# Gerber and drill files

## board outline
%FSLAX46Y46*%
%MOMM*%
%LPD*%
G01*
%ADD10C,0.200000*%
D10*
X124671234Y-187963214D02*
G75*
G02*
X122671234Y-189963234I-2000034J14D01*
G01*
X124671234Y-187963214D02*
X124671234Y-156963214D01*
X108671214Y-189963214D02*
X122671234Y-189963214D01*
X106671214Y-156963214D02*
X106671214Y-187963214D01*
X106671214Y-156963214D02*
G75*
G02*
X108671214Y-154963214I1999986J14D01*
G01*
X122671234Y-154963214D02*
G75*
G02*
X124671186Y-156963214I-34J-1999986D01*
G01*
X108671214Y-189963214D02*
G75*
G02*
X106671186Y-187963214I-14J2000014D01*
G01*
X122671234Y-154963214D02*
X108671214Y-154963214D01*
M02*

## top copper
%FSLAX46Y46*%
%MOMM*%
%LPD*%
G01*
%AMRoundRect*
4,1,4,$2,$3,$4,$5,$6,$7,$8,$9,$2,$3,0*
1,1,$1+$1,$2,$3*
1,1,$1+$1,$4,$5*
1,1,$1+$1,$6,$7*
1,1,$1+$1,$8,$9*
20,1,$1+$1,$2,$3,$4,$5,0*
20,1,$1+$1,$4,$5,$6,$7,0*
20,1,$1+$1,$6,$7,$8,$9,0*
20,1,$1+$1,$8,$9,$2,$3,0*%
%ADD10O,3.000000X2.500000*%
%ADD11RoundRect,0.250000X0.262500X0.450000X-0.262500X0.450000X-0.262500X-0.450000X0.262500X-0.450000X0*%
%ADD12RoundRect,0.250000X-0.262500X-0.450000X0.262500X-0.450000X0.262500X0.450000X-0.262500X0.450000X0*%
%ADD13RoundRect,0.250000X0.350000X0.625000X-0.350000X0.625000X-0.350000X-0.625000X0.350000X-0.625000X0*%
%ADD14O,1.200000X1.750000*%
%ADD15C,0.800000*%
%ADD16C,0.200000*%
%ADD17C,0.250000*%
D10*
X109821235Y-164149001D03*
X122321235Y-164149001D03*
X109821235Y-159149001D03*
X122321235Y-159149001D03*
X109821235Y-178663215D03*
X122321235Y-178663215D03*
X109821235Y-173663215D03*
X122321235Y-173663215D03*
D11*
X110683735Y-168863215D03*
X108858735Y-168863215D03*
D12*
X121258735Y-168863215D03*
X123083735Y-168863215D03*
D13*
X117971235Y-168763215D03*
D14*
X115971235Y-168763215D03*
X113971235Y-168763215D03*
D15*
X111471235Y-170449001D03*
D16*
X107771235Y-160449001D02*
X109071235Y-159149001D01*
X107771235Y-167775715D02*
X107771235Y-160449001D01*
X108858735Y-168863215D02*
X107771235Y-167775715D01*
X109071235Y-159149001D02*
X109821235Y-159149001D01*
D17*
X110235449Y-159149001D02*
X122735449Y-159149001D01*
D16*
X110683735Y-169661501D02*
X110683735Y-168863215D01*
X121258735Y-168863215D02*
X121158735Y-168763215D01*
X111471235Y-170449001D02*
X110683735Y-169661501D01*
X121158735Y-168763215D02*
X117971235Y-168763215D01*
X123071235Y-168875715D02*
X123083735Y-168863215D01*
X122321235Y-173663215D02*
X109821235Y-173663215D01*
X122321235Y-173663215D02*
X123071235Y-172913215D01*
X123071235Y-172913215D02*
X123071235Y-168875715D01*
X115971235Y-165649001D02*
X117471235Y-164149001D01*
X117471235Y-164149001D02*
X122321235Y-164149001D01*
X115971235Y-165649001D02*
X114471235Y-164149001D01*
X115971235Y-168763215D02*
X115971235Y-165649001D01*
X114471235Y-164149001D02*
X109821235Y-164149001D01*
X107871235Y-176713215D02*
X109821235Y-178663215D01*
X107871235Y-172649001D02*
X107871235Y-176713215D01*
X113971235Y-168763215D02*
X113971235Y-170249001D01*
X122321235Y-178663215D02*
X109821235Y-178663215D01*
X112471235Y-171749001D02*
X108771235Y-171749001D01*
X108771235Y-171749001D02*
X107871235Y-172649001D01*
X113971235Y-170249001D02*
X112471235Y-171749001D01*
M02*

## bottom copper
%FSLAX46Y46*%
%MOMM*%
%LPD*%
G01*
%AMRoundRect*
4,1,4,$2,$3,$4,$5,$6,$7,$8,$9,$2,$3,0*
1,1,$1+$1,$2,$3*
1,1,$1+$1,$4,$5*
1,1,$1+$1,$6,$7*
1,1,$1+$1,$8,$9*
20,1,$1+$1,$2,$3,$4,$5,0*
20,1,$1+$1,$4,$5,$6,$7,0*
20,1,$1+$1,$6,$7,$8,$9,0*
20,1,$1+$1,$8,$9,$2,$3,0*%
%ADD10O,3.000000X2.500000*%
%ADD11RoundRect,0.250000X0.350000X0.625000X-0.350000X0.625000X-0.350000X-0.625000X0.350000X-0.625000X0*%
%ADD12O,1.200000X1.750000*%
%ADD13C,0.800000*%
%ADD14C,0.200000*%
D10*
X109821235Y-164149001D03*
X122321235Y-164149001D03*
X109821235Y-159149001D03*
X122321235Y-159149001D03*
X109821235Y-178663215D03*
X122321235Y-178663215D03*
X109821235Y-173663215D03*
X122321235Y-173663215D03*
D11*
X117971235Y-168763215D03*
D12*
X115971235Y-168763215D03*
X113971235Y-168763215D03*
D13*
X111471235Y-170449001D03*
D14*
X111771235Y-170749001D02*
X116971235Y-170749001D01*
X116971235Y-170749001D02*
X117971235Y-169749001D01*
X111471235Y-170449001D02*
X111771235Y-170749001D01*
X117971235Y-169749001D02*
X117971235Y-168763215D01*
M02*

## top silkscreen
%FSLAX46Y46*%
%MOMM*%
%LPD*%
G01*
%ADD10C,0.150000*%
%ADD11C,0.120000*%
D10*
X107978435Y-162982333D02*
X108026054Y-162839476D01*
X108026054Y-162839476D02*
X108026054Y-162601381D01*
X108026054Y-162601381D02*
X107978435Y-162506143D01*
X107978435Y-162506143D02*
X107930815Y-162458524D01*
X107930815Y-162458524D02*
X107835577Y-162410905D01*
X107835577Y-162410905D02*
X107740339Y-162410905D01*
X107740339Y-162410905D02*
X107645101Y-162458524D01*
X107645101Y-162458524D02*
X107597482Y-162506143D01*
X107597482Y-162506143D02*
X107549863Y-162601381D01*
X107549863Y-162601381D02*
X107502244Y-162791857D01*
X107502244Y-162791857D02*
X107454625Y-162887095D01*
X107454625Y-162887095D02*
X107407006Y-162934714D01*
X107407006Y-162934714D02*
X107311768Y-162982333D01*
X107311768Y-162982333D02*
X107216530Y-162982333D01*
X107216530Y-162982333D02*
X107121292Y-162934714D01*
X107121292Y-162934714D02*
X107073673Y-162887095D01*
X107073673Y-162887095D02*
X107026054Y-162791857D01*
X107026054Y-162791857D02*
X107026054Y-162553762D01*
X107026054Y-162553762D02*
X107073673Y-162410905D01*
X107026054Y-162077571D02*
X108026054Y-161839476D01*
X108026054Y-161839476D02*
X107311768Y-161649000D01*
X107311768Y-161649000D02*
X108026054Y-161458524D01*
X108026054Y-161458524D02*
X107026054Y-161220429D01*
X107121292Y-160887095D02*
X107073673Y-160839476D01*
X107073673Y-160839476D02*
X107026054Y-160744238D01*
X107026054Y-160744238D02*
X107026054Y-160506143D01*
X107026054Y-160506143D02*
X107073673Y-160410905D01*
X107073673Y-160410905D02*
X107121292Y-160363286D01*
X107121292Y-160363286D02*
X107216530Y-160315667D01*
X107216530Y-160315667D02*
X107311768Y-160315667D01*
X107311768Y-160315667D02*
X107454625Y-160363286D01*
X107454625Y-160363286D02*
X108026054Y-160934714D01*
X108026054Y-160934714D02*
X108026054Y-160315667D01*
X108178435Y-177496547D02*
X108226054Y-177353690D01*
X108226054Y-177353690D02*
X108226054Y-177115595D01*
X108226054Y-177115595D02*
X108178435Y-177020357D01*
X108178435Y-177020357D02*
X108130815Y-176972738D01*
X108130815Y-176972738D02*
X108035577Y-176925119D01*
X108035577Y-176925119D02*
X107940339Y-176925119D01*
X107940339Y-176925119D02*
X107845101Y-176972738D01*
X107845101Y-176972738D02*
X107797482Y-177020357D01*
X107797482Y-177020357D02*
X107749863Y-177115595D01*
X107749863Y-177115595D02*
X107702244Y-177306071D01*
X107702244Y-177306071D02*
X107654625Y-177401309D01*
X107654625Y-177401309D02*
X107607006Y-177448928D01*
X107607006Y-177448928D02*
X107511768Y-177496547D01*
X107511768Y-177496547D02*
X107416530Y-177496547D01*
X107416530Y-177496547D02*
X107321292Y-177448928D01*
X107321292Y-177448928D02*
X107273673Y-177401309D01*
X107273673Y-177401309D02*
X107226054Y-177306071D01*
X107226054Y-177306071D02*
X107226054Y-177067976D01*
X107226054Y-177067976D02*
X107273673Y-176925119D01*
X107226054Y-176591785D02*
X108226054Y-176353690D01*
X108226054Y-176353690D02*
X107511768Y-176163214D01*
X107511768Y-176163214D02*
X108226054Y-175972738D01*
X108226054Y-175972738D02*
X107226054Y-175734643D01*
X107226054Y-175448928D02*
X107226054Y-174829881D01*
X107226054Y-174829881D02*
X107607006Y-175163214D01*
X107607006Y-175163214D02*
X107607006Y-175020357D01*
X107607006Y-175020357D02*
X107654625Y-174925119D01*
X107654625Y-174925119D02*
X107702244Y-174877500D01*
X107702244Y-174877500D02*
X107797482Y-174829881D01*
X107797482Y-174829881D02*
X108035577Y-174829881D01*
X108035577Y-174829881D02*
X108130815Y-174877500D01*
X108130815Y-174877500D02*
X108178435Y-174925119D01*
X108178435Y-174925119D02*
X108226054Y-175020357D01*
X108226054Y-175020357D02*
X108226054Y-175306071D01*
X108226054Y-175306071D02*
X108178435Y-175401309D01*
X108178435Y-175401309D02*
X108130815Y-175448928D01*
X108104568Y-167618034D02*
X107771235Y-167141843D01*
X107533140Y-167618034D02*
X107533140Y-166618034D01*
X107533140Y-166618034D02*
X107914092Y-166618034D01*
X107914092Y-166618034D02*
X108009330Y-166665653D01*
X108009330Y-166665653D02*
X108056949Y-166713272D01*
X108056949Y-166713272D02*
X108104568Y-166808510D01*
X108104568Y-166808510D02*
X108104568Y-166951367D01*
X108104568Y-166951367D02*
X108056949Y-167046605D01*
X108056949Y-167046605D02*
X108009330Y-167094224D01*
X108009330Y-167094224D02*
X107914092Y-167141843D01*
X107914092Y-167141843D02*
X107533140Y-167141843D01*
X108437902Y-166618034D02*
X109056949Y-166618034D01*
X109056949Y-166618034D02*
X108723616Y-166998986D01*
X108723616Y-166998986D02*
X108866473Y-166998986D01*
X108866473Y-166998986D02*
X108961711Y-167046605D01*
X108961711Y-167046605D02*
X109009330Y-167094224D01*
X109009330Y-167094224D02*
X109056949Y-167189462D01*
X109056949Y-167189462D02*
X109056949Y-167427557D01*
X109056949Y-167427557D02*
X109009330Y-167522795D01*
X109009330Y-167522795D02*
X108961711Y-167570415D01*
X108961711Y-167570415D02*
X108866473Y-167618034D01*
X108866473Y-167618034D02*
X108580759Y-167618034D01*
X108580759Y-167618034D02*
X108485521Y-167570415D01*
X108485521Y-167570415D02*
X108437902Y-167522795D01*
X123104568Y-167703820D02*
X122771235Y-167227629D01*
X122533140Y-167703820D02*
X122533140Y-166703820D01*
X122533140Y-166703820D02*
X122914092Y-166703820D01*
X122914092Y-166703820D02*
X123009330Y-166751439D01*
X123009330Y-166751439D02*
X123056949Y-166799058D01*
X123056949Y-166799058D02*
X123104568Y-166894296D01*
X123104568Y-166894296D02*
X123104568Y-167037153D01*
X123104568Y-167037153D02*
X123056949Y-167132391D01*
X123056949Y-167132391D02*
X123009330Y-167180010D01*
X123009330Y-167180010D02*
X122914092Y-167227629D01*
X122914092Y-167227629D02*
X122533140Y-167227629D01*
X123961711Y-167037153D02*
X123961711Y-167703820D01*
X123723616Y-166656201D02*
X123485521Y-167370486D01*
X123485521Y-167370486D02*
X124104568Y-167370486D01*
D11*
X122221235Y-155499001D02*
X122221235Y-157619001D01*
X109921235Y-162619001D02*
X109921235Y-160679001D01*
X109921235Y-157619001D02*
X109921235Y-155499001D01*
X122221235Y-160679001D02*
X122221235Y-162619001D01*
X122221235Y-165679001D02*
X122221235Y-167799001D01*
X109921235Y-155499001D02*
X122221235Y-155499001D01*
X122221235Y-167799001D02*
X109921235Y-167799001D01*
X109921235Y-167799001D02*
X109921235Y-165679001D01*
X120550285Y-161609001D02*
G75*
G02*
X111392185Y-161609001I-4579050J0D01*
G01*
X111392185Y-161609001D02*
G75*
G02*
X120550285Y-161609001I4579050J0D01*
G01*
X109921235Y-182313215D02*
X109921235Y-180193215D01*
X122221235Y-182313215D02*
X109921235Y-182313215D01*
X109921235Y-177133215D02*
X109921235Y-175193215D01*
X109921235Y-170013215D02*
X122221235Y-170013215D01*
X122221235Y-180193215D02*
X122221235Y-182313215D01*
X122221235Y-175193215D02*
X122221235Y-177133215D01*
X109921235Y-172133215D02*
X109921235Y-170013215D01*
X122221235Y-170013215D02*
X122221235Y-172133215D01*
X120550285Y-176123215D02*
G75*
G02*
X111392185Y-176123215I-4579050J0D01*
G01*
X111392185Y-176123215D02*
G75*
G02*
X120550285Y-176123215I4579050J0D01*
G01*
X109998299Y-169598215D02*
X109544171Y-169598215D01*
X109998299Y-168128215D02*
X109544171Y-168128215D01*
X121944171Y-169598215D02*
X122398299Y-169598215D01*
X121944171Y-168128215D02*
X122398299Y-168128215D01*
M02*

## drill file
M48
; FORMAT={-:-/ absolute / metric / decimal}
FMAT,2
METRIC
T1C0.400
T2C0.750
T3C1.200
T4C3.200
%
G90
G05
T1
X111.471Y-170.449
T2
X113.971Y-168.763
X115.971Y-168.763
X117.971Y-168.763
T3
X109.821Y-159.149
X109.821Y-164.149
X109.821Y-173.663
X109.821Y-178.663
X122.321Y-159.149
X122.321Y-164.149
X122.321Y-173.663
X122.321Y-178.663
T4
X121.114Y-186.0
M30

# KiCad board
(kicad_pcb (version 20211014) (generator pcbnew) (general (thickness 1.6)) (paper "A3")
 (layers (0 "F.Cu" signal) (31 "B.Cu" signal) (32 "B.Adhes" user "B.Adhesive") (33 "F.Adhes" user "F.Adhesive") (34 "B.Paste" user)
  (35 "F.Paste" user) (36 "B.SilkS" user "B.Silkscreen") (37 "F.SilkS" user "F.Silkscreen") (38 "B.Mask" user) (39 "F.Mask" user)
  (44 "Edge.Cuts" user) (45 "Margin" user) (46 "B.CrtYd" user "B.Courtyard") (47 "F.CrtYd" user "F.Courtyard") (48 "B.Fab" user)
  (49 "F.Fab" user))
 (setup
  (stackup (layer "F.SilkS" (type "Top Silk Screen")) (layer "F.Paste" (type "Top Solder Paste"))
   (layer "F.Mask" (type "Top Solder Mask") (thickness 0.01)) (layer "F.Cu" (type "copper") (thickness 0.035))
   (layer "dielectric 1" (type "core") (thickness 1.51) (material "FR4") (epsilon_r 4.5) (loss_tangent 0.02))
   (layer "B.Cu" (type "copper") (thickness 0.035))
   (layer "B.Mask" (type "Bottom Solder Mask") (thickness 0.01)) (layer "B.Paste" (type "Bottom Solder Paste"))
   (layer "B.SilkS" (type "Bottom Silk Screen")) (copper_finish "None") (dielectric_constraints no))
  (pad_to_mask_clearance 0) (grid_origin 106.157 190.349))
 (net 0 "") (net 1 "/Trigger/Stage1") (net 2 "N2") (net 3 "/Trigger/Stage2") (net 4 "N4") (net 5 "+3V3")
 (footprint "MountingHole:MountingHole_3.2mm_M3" (layer "F.Cu") (at 121.114235 186.000001)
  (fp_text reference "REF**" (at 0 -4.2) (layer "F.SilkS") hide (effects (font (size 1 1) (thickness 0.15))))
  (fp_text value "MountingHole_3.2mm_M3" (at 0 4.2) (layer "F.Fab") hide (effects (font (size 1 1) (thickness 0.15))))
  (pad "" np_thru_hole circle (at 0 0) (size 3.2 3.2) (drill 3.2) (layers F&B.Cu *.Mask)))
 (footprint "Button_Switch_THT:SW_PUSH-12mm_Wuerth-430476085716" (layer "F.Cu") (at 122.321235 164.149001 180)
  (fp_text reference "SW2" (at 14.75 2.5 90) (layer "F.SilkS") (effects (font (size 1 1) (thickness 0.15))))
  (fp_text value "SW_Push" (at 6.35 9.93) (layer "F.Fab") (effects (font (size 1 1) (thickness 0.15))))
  (fp_line (start 0.1 8.65) (end 0.1 6.53) (layer "F.SilkS") (width 0.12))
  (fp_line (start 12.4 1.53) (end 12.4 3.47) (layer "F.SilkS") (width 0.12))
  (fp_line (start 12.4 6.53) (end 12.4 8.65) (layer "F.SilkS") (width 0.12))
  (fp_line (start 0.1 3.47) (end 0.1 1.53) (layer "F.SilkS") (width 0.12))
  (fp_line (start 0.1 -1.53) (end 0.1 -3.65) (layer "F.SilkS") (width 0.12))
  (fp_line (start 12.4 8.65) (end 0.1 8.65) (layer "F.SilkS") (width 0.12))
  (fp_line (start 0.1 -3.65) (end 12.4 -3.65) (layer "F.SilkS") (width 0.12))
  (fp_line (start 12.4 -3.65) (end 12.4 -1.53) (layer "F.SilkS") (width 0.12))
  (fp_circle (center 6.35 2.54) (end 10.92905 2.54) (layer "F.SilkS") (width 0.12) (fill none))
  (pad "1" thru_hole oval (at 12.5 0 180) (size 3 2.5) (drill 1.2) (layers F&B.Cu *.Mask) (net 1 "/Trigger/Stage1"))
  (pad "1" thru_hole oval (at 0 0 180) (size 3 2.5) (drill 1.2) (layers F&B.Cu *.Mask) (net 1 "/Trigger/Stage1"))
  (pad "2" thru_hole oval (at 12.5 5 180) (size 3 2.5) (drill 1.2) (layers F&B.Cu *.Mask) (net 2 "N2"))
  (pad "2" thru_hole oval (at 0 5 180) (size 3 2.5) (drill 1.2) (layers F&B.Cu *.Mask) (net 2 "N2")))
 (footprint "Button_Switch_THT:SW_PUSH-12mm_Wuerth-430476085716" (layer "F.Cu") (at 122.321235 178.663215 180)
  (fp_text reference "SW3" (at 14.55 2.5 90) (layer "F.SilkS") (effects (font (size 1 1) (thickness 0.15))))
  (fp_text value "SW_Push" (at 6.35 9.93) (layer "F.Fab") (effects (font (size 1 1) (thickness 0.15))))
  (fp_line (start 12.4 -3.65) (end 12.4 -1.53) (layer "F.SilkS") (width 0.12))
  (fp_line (start 0.1 -3.65) (end 12.4 -3.65) (layer "F.SilkS") (width 0.12))
  (fp_line (start 12.4 1.53) (end 12.4 3.47) (layer "F.SilkS") (width 0.12))
  (fp_line (start 12.4 8.65) (end 0.1 8.65) (layer "F.SilkS") (width 0.12))
  (fp_line (start 0.1 -1.53) (end 0.1 -3.65) (layer "F.SilkS") (width 0.12))
  (fp_line (start 0.1 3.47) (end 0.1 1.53) (layer "F.SilkS") (width 0.12))
  (fp_line (start 12.4 6.53) (end 12.4 8.65) (layer "F.SilkS") (width 0.12))
  (fp_line (start 0.1 8.65) (end 0.1 6.53) (layer "F.SilkS") (width 0.12))
  (fp_circle (center 6.35 2.54) (end 10.92905 2.54) (layer "F.SilkS") (width 0.12) (fill none))
  (pad "1" thru_hole oval (at 12.5 0 180) (size 3 2.5) (drill 1.2) (layers F&B.Cu *.Mask) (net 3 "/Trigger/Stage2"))
  (pad "1" thru_hole oval (at 0 0 180) (size 3 2.5) (drill 1.2) (layers F&B.Cu *.Mask) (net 3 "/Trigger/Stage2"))
  (pad "2" thru_hole oval (at 12.5 5 180) (size 3 2.5) (drill 1.2) (layers F&B.Cu *.Mask) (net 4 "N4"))
  (pad "2" thru_hole oval (at 0 5 180) (size 3 2.5) (drill 1.2) (layers F&B.Cu *.Mask) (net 4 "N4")))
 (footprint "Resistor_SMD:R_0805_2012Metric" (layer "F.Cu") (at 109.771235 168.863215 180)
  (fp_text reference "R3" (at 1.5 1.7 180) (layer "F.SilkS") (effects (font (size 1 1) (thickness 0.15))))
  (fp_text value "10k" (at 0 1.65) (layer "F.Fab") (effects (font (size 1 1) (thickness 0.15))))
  (fp_line (start -0.227064 -0.735) (end 0.227064 -0.735) (layer "F.SilkS") (width 0.12))
  (fp_line (start -0.227064 0.735) (end 0.227064 0.735) (layer "F.SilkS") (width 0.12))
  (pad "1" smd roundrect (at -0.9125 0 180) (size 1.025 1.4) (layers "F.Cu" "F.Paste" "F.Mask") (roundrect_rratio 0.243902) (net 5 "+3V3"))
  (pad "2" smd roundrect (at 0.9125 0 180) (size 1.025 1.4) (layers "F.Cu" "F.Paste" "F.Mask") (roundrect_rratio 0.243902) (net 2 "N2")))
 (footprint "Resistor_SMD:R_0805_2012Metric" (layer "F.Cu") (at 122.171235 168.863215)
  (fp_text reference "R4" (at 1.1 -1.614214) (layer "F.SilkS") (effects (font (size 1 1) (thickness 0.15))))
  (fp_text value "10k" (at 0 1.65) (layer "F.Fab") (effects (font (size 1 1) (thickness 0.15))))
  (fp_line (start -0.227064 0.735) (end 0.227064 0.735) (layer "F.SilkS") (width 0.12))
  (fp_line (start -0.227064 -0.735) (end 0.227064 -0.735) (layer "F.SilkS") (width 0.12))
  (pad "1" smd roundrect (at -0.9125 0) (size 1.025 1.4) (layers "F.Cu" "F.Paste" "F.Mask") (roundrect_rratio 0.243902) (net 5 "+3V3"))
  (pad "2" smd roundrect (at 0.9125 0) (size 1.025 1.4) (layers "F.Cu" "F.Paste" "F.Mask") (roundrect_rratio 0.243902) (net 4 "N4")))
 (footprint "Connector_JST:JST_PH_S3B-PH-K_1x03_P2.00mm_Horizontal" (layer "B.Cu") (at 117.971235 168.763215 180)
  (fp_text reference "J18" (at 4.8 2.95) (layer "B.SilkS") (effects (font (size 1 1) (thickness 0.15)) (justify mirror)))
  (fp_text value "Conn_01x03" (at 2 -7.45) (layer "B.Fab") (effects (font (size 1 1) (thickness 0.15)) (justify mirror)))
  (pad "1" thru_hole roundrect (at 0 0 180) (size 1.2 1.75) (drill 0.75) (layers F&B.Cu *.Mask) (roundrect_rratio 0.208333) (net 5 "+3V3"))
  (pad "2" thru_hole oval (at 2 0 180) (size 1.2 1.75) (drill 0.75) (layers F&B.Cu *.Mask) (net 1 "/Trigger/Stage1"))
  (pad "3" thru_hole oval (at 4 0 180) (size 1.2 1.75) (drill 0.75) (layers F&B.Cu *.Mask) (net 3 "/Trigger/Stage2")))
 (gr_arc (start 124.671234 187.963214) (mid 124.085445 189.377431) (end 122.671234 189.963214) (layer "Edge.Cuts") (width 0.2))
 (gr_line (start 124.671234 187.963214) (end 124.671234 156.963214) (layer "Edge.Cuts") (width 0.2))
 (gr_line (start 108.671214 189.963214) (end 122.671234 189.963214) (layer "Edge.Cuts") (width 0.2))
 (gr_line (start 106.671214 156.963214) (end 106.671214 187.963214) (layer "Edge.Cuts") (width 0.2))
 (gr_arc (start 106.671214 156.963214) (mid 107.25699 155.54899) (end 108.671214 154.963214) (layer "Edge.Cuts") (width 0.2))
 (gr_arc (start 122.671234 154.963214) (mid 124.085447 155.549001) (end 124.671234 156.963214) (layer "Edge.Cuts") (width 0.2))
 (gr_arc (start 108.671214 189.963214) (mid 107.257009 189.37742) (end 106.671214 187.963214) (layer "Edge.Cuts") (width 0.2))
 (gr_line (start 122.671234 154.963214) (end 108.671214 154.963214) (layer "Edge.Cuts") (width 0.2))
 (segment (start 107.771235 160.449001) (end 109.071235 159.149001) (width 0.2) (layer "F.Cu") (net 2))
 (segment (start 107.771235 167.775715) (end 107.771235 160.449001) (width 0.2) (layer "F.Cu") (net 2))
 (segment (start 108.858735 168.863215) (end 107.771235 167.775715) (width 0.2) (layer "F.Cu") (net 2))
 (segment (start 109.071235 159.149001) (end 109.821235 159.149001) (width 0.2) (layer "F.Cu") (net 2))
 (segment (start 110.235449 159.149001) (end 122.735449 159.149001) (width 0.25) (layer "F.Cu") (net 2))
 (segment (start 110.683735 169.661501) (end 110.683735 168.863215) (width 0.2) (layer "F.Cu") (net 5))
 (segment (start 121.258735 168.863215) (end 121.158735 168.763215) (width 0.2) (layer "F.Cu") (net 5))
 (segment (start 111.471235 170.449001) (end 110.683735 169.661501) (width 0.2) (layer "F.Cu") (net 5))
 (segment (start 121.158735 168.763215) (end 117.971235 168.763215) (width 0.2) (layer "F.Cu") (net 5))
 (via (at 111.471235 170.449001) (size 0.8) (drill 0.4) (layers "F.Cu" "B.Cu") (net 5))
 (segment (start 111.771235 170.749001) (end 116.971235 170.749001) (width 0.2) (layer "B.Cu") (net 5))
 (segment (start 116.971235 170.749001) (end 117.971235 169.749001) (width 0.2) (layer "B.Cu") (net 5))
 (segment (start 111.471235 170.449001) (end 111.771235 170.749001) (width 0.2) (layer "B.Cu") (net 5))
 (segment (start 117.971235 169.749001) (end 117.971235 168.763215) (width 0.2) (layer "B.Cu") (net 5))
 (segment (start 123.071235 168.875715) (end 123.083735 168.863215) (width 0.2) (layer "F.Cu") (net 4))
 (segment (start 122.321235 173.663215) (end 109.821235 173.663215) (width 0.2) (layer "F.Cu") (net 4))
 (segment (start 122.321235 173.663215) (end 123.071235 172.913215) (width 0.2) (layer "F.Cu") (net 4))
 (segment (start 123.071235 172.913215) (end 123.071235 168.875715) (width 0.2) (layer "F.Cu") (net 4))
 (segment (start 115.971235 165.649001) (end 117.471235 164.149001) (width 0.2) (layer "F.Cu") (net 1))
 (segment (start 117.471235 164.149001) (end 122.321235 164.149001) (width 0.2) (layer "F.Cu") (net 1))
 (segment (start 115.971235 165.649001) (end 114.471235 164.149001) (width 0.2) (layer "F.Cu") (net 1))
 (segment (start 115.971235 168.763215) (end 115.971235 165.649001) (width 0.2) (layer "F.Cu") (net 1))
 (segment (start 114.471235 164.149001) (end 109.821235 164.149001) (width 0.2) (layer "F.Cu") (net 1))
 (segment (start 107.871235 176.713215) (end 109.821235 178.663215) (width 0.2) (layer "F.Cu") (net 3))
 (segment (start 107.871235 172.649001) (end 107.871235 176.713215) (width 0.2) (layer "F.Cu") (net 3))
 (segment (start 113.971235 168.763215) (end 113.971235 170.249001) (width 0.2) (layer "F.Cu") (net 3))
 (segment (start 122.321235 178.663215) (end 109.821235 178.663215) (width 0.2) (layer "F.Cu") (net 3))
 (segment (start 112.471235 171.749001) (end 108.771235 171.749001) (width 0.2) (layer "F.Cu") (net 3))
 (segment (start 108.771235 171.749001) (end 107.871235 172.649001) (width 0.2) (layer "F.Cu") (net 3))
 (segment (start 113.971235 170.249001) (end 112.471235 171.749001) (width 0.2) (layer "F.Cu") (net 3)))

